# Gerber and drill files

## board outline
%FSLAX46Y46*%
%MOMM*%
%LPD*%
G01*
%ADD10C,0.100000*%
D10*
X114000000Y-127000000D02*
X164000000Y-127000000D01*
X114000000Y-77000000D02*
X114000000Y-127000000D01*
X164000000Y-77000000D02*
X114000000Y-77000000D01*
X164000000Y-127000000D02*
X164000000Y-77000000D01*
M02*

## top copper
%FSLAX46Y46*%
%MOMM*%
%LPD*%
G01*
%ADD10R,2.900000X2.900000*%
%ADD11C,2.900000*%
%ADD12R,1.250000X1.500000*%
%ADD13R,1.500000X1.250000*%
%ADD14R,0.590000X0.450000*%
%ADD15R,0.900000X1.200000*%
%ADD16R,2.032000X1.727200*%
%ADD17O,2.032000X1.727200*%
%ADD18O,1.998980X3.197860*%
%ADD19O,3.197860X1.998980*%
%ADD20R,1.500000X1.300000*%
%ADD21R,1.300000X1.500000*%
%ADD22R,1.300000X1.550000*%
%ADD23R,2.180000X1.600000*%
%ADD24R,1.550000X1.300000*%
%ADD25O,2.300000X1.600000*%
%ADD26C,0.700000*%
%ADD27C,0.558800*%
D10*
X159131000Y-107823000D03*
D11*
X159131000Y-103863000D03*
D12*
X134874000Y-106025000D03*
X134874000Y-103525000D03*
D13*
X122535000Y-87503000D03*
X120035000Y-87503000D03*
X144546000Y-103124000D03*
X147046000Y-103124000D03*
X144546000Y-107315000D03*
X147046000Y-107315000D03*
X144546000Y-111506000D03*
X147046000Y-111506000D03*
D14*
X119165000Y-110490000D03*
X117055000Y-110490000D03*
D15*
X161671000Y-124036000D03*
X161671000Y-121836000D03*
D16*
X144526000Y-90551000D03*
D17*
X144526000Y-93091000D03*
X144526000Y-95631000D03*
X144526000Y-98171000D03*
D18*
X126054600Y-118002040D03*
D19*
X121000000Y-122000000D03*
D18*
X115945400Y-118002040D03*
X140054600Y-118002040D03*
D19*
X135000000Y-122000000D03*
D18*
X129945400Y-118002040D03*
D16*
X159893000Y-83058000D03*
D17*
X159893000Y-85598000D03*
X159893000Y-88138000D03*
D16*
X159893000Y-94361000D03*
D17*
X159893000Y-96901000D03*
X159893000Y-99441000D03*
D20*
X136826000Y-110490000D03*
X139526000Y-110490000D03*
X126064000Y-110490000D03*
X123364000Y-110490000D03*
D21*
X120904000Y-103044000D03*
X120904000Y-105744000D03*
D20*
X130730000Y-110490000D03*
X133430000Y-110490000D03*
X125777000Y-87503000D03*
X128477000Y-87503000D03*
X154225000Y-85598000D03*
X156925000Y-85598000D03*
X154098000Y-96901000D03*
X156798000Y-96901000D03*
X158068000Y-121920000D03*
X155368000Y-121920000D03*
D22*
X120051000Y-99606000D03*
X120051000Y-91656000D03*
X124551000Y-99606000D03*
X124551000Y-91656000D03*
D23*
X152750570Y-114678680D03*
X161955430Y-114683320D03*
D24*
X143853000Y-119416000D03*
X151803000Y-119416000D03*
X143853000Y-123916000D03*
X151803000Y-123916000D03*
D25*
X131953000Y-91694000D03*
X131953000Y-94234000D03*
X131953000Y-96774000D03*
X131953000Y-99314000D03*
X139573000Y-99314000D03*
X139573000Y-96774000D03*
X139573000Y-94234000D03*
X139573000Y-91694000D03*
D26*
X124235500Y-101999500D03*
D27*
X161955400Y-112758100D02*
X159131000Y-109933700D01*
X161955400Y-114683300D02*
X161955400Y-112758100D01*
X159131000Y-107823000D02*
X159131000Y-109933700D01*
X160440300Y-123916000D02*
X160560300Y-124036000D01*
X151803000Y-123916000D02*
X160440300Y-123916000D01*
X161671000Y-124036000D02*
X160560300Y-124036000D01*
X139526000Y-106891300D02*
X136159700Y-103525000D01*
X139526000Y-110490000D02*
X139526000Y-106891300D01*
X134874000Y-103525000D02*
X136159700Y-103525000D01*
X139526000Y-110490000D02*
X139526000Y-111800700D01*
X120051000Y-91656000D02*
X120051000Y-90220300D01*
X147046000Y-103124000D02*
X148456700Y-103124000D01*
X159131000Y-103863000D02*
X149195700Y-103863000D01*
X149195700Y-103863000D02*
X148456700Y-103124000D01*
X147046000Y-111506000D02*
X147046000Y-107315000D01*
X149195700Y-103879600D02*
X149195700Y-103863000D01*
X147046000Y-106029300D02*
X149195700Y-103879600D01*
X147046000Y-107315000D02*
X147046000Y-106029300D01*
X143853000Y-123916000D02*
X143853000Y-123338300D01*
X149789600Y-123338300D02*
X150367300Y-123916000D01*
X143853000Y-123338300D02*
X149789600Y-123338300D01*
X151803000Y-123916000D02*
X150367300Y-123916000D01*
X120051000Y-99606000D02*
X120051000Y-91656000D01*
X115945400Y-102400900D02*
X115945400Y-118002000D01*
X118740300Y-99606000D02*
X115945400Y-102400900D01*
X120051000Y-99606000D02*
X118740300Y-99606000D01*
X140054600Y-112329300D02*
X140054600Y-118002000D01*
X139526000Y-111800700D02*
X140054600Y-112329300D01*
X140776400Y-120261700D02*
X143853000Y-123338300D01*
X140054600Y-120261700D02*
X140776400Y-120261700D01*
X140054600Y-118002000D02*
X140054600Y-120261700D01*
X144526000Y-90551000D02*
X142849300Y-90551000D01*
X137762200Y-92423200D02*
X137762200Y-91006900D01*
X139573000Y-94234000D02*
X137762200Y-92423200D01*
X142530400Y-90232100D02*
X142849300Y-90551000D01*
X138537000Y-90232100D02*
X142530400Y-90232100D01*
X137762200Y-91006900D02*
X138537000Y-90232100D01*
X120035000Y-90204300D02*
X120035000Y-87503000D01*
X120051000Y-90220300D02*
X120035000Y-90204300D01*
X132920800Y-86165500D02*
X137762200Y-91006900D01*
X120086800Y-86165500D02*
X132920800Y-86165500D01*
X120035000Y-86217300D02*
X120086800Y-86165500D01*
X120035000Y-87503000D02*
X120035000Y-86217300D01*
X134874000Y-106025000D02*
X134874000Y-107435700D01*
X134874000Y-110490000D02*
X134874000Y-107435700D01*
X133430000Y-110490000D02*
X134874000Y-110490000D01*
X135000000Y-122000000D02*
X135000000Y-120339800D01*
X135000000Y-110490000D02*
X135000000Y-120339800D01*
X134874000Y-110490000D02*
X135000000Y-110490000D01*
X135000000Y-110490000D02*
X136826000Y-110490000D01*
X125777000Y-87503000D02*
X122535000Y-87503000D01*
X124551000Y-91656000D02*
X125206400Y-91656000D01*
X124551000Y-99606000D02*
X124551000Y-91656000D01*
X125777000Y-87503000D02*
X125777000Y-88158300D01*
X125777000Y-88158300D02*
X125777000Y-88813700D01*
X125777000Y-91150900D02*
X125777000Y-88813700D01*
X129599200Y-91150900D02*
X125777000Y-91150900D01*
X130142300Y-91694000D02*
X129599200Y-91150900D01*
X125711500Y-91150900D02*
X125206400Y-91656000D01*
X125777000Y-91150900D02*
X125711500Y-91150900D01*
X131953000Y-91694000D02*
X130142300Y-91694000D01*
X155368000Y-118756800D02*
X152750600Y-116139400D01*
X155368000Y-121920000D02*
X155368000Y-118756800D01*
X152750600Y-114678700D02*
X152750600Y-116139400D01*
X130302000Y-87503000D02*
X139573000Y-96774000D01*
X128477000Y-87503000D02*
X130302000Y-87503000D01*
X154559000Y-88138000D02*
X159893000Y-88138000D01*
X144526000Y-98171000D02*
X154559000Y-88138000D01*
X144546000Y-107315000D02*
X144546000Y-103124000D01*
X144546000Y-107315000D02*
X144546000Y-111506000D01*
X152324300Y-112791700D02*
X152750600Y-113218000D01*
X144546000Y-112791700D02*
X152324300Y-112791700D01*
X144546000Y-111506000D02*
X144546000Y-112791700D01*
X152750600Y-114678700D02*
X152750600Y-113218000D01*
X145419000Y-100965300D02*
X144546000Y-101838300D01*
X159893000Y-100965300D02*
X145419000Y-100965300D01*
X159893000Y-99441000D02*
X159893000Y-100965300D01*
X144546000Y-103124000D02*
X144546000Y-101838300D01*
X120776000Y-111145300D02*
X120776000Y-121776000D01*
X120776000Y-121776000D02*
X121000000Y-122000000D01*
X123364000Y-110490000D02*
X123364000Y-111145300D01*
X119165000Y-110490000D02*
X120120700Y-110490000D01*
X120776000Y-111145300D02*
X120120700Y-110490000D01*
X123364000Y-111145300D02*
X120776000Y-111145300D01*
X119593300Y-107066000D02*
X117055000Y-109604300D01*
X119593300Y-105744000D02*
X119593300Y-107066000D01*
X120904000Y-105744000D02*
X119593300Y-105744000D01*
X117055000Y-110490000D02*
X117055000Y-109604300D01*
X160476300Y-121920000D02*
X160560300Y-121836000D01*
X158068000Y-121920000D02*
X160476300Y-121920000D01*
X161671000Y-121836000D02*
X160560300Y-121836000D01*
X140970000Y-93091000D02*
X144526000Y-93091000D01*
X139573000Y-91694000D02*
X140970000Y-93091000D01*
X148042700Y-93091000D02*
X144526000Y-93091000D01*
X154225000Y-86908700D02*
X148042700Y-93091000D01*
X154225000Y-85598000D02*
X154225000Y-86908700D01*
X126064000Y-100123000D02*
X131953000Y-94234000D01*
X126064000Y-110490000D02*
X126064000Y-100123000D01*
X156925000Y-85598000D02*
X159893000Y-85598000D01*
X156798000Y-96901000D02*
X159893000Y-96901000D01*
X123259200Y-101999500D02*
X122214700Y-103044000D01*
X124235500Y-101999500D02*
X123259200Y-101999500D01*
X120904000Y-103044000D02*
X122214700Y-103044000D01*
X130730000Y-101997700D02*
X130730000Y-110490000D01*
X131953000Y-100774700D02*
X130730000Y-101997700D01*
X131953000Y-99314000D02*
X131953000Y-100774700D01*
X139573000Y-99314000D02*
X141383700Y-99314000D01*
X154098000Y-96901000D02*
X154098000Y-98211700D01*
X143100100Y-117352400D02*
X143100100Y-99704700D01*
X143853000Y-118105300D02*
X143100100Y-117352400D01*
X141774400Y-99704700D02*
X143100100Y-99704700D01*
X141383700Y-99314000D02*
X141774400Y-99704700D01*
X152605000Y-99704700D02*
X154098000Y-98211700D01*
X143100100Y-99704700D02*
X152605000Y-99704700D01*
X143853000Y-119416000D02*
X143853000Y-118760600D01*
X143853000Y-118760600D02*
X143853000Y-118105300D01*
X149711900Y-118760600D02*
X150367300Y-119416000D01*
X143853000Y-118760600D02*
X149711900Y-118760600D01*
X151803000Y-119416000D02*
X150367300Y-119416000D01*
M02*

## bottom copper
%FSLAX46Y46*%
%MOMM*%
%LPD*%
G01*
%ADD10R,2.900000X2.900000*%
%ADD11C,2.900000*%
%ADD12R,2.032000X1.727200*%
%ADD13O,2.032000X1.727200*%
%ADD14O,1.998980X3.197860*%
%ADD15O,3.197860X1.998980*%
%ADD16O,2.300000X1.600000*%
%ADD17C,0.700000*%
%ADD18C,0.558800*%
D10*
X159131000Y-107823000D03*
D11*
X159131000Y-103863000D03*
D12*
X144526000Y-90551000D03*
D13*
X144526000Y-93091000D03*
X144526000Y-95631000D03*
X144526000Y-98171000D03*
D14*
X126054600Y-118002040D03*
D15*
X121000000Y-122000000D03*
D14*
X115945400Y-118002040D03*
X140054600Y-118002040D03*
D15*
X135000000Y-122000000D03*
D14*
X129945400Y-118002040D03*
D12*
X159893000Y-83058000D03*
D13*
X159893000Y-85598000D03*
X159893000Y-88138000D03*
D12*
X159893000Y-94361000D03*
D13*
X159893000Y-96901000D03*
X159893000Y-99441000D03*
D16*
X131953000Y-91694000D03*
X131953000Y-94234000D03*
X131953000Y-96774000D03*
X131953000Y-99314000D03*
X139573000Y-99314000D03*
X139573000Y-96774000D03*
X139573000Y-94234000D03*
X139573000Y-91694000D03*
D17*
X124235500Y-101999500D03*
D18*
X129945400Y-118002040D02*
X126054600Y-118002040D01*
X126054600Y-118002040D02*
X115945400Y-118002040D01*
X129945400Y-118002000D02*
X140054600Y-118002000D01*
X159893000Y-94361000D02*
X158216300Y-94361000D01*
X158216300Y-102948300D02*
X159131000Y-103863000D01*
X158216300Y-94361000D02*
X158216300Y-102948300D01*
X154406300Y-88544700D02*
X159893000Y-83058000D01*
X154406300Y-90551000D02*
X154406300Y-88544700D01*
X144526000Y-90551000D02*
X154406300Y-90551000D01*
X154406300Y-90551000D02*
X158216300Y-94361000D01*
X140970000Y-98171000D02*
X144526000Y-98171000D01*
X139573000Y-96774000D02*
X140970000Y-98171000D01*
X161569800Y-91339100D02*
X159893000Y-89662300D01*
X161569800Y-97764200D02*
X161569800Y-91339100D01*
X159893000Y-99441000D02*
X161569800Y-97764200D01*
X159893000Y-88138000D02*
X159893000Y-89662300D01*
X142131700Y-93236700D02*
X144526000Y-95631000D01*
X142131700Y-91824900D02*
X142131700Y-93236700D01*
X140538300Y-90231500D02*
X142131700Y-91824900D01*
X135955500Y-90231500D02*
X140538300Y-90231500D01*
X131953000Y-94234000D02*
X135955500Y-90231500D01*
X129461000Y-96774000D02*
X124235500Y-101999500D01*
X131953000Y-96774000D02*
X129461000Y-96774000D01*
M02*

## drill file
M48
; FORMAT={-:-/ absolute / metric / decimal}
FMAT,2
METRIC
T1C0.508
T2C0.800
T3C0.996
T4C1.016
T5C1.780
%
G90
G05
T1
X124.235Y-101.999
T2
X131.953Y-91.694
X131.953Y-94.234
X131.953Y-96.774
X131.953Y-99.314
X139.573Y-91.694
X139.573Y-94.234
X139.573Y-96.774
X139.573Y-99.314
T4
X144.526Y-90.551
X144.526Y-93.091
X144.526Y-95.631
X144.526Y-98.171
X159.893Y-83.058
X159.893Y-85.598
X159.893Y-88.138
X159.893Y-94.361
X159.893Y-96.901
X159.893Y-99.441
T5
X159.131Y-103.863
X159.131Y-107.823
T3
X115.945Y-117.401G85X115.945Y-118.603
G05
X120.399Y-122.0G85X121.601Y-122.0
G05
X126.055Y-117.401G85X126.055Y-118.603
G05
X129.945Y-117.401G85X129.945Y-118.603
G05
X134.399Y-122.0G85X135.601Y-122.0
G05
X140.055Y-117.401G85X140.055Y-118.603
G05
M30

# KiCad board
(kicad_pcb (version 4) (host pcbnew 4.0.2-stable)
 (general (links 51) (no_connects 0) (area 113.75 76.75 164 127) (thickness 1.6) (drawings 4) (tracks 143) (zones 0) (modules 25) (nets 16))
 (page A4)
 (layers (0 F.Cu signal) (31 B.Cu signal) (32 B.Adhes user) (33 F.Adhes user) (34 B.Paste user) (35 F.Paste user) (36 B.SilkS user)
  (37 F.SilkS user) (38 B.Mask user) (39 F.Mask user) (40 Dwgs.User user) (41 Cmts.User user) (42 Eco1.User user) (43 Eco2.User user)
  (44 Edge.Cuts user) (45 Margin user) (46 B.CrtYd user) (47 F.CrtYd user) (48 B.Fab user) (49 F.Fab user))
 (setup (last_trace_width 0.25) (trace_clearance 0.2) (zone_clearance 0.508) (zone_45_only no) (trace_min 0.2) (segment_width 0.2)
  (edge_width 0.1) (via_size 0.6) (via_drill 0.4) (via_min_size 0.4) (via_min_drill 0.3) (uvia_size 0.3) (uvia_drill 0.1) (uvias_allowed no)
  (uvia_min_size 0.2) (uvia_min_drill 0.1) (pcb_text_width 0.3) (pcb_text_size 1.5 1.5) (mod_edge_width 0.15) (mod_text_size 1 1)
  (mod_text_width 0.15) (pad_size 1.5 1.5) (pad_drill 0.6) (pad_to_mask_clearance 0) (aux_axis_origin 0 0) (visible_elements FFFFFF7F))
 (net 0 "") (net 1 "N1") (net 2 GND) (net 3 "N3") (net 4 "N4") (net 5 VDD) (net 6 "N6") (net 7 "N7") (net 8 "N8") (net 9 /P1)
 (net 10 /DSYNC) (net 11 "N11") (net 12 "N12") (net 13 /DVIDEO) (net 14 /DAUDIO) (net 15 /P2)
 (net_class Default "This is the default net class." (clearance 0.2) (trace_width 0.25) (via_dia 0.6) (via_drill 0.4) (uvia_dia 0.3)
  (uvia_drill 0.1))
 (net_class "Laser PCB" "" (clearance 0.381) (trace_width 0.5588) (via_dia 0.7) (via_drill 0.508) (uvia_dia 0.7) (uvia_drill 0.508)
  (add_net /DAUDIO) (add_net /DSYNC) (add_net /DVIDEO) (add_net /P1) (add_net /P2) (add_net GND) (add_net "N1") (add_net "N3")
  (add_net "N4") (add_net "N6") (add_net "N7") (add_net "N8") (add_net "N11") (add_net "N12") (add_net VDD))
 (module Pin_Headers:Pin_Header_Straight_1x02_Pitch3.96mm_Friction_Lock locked (layer F.Cu) (at 159.131 107.823 90)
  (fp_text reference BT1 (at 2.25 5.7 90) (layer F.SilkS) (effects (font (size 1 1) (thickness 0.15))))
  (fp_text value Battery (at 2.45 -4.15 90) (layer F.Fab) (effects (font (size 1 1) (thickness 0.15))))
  (pad 1 thru_hole rect (at 0 0 90) (size 2.9 2.9) (drill 1.78) (layers *.Cu *.Mask F.SilkS) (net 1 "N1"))
  (pad 2 thru_hole circle (at 3.96 0 90) (size 2.9 2.9) (drill 1.78) (layers *.Cu *.Mask F.SilkS) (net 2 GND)))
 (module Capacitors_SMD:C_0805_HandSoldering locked (layer F.Cu) (at 134.874 104.775 90)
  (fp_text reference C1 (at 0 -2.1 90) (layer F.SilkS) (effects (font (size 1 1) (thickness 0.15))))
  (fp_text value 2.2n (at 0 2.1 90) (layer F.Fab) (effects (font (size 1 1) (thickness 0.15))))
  (pad 1 smd rect (at -1.25 0 90) (size 1.5 1.25) (layers F.Cu F.Paste F.Mask) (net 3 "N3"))
  (pad 2 smd rect (at 1.25 0 90) (size 1.5 1.25) (layers F.Cu F.Paste F.Mask) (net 2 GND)))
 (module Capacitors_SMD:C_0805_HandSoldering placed (layer F.Cu) (at 121.285 87.503 180)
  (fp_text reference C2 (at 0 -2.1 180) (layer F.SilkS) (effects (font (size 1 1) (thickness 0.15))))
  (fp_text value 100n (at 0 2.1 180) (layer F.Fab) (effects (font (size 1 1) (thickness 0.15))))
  (pad 1 smd rect (at -1.25 0 180) (size 1.5 1.25) (layers F.Cu F.Paste F.Mask) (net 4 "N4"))
  (pad 2 smd rect (at 1.25 0 180) (size 1.5 1.25) (layers F.Cu F.Paste F.Mask) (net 2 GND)))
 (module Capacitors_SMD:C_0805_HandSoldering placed (layer F.Cu) (at 145.796 103.124)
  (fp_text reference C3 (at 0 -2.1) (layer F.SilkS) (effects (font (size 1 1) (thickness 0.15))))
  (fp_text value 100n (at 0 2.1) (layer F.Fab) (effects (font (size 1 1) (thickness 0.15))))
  (pad 1 smd rect (at -1.25 0) (size 1.5 1.25) (layers F.Cu F.Paste F.Mask) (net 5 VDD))
  (pad 2 smd rect (at 1.25 0) (size 1.5 1.25) (layers F.Cu F.Paste F.Mask) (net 2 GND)))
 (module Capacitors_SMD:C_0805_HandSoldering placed (layer F.Cu) (at 145.796 107.315)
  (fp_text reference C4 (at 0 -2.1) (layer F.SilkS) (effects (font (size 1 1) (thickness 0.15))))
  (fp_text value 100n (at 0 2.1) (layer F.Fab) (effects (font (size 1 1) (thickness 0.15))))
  (pad 1 smd rect (at -1.25 0) (size 1.5 1.25) (layers F.Cu F.Paste F.Mask) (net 5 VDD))
  (pad 2 smd rect (at 1.25 0) (size 1.5 1.25) (layers F.Cu F.Paste F.Mask) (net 2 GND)))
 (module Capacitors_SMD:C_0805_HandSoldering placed (layer F.Cu) (at 145.796 111.506)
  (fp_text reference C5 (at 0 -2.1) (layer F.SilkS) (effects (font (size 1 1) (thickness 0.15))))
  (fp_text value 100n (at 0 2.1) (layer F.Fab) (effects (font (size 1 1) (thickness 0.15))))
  (pad 1 smd rect (at -1.25 0) (size 1.5 1.25) (layers F.Cu F.Paste F.Mask) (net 5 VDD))
  (pad 2 smd rect (at 1.25 0) (size 1.5 1.25) (layers F.Cu F.Paste F.Mask) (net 2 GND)))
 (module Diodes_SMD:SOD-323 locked (layer F.Cu) (at 118.11 110.49 180)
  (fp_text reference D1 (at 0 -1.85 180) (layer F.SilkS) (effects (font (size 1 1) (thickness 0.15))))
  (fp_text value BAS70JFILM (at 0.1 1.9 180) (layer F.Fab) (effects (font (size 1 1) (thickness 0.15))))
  (pad 1 smd rect (at -1.055 0 180) (size 0.59 0.45) (layers F.Cu F.Paste F.Mask) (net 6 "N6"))
  (pad 2 smd rect (at 1.055 0 180) (size 0.59 0.45) (layers F.Cu F.Paste F.Mask) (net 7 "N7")))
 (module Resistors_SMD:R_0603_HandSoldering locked (layer F.Cu) (at 161.671 122.936 90)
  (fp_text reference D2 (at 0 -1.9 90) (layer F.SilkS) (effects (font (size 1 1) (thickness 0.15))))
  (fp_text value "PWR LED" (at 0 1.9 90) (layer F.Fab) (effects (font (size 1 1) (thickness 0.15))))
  (pad 1 smd rect (at -1.1 0 90) (size 1.2 0.9) (layers F.Cu F.Paste F.Mask) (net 2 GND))
  (pad 2 smd rect (at 1.1 0 90) (size 1.2 0.9) (layers F.Cu F.Paste F.Mask) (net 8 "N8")))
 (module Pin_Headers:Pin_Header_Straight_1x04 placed (layer F.Cu) (at 144.526 90.551)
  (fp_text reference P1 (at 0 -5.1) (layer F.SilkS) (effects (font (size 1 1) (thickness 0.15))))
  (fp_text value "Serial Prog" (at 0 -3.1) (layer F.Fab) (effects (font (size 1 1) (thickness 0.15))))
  (pad 1 thru_hole rect (at 0 0) (size 2.032 1.7272) (drill 1.016) (layers *.Cu *.Mask F.SilkS) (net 2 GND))
  (pad 2 thru_hole oval (at 0 2.54) (size 2.032 1.7272) (drill 1.016) (layers *.Cu *.Mask F.SilkS) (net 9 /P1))
  (pad 3 thru_hole oval (at 0 5.08) (size 2.032 1.7272) (drill 1.016) (layers *.Cu *.Mask F.SilkS) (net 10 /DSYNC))
  (pad 4 thru_hole oval (at 0 7.62) (size 2.032 1.7272) (drill 1.016) (layers *.Cu *.Mask F.SilkS) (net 5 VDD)))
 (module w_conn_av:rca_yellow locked (layer F.Cu) (at 121 122)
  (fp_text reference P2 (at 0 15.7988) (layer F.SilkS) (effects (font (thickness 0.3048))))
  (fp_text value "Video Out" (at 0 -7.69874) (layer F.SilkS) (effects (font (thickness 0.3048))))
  (pad 2 thru_hole oval (at 5.0546 -3.99796) (size 1.99898 3.19786) (drill oval 0.99568 2.1971) (layers *.Cu *.Mask F.SilkS) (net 2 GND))
  (pad 1 thru_hole oval (at 0 0) (size 3.19786 1.99898) (drill oval 2.1971 0.99568) (layers *.Cu *.Mask F.SilkS) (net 6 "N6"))
  (pad 2 thru_hole oval (at -5.0546 -3.99796) (size 1.99898 3.19786) (drill oval 0.99568 2.1971) (layers *.Cu *.Mask F.SilkS) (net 2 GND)))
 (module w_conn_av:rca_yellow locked (layer F.Cu) (at 135 122)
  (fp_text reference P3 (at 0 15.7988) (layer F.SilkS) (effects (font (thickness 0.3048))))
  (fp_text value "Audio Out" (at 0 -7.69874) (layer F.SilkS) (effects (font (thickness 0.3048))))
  (pad 2 thru_hole oval (at 5.0546 -3.99796) (size 1.99898 3.19786) (drill oval 0.99568 2.1971) (layers *.Cu *.Mask F.SilkS) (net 2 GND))
  (pad 1 thru_hole oval (at 0 0) (size 3.19786 1.99898) (drill oval 2.1971 0.99568) (layers *.Cu *.Mask F.SilkS) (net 3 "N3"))
  (pad 2 thru_hole oval (at -5.0546 -3.99796) (size 1.99898 3.19786) (drill oval 0.99568 2.1971) (layers *.Cu *.Mask F.SilkS) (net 2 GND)))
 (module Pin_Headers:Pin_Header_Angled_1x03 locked (layer F.Cu) (at 159.893 83.058)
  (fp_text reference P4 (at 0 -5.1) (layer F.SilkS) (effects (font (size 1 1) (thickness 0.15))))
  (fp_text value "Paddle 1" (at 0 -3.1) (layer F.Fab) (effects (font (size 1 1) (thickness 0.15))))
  (pad 1 thru_hole rect (at 0 0) (size 2.032 1.7272) (drill 1.016) (layers *.Cu *.Mask F.SilkS) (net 2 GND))
  (pad 2 thru_hole oval (at 0 2.54) (size 2.032 1.7272) (drill 1.016) (layers *.Cu *.Mask F.SilkS) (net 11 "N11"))
  (pad 3 thru_hole oval (at 0 5.08) (size 2.032 1.7272) (drill 1.016) (layers *.Cu *.Mask F.SilkS) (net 5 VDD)))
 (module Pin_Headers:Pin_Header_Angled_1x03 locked (layer F.Cu) (at 159.893 94.361)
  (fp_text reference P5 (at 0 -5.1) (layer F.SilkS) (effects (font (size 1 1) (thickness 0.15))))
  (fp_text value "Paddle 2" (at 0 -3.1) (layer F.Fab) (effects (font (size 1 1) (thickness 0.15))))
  (pad 1 thru_hole rect (at 0 0) (size 2.032 1.7272) (drill 1.016) (layers *.Cu *.Mask F.SilkS) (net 2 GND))
  (pad 2 thru_hole oval (at 0 2.54) (size 2.032 1.7272) (drill 1.016) (layers *.Cu *.Mask F.SilkS) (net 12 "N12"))
  (pad 3 thru_hole oval (at 0 5.08) (size 2.032 1.7272) (drill 1.016) (layers *.Cu *.Mask F.SilkS) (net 5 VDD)))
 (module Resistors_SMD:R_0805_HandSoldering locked (layer F.Cu) (at 138.176 110.49)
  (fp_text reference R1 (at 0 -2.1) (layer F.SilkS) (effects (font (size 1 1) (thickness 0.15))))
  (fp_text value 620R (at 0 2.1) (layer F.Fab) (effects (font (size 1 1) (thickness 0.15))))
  (pad 1 smd rect (at -1.35 0) (size 1.5 1.3) (layers F.Cu F.Paste F.Mask) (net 3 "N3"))
  (pad 2 smd rect (at 1.35 0) (size 1.5 1.3) (layers F.Cu F.Paste F.Mask) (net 2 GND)))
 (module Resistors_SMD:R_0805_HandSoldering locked (layer F.Cu) (at 124.714 110.49 180)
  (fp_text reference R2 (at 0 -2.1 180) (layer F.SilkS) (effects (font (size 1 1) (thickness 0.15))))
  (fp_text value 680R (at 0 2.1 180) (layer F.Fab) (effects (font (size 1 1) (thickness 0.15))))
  (pad 1 smd rect (at -1.35 0 180) (size 1.5 1.3) (layers F.Cu F.Paste F.Mask) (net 10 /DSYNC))
  (pad 2 smd rect (at 1.35 0 180) (size 1.5 1.3) (layers F.Cu F.Paste F.Mask) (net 6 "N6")))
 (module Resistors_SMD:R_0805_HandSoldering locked (layer F.Cu) (at 120.904 104.394 270)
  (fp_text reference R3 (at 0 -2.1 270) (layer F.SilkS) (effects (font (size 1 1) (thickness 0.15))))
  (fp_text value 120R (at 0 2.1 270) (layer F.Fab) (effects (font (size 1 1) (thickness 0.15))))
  (pad 1 smd rect (at -1.35 0 270) (size 1.5 1.3) (layers F.Cu F.Paste F.Mask) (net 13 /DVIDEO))
  (pad 2 smd rect (at 1.35 0 270) (size 1.5 1.3) (layers F.Cu F.Paste F.Mask) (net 7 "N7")))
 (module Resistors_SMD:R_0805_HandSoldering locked (layer F.Cu) (at 132.08 110.49)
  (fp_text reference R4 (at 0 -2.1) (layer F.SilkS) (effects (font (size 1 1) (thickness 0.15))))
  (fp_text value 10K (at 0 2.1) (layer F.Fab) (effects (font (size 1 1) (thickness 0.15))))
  (pad 1 smd rect (at -1.35 0) (size 1.5 1.3) (layers F.Cu F.Paste F.Mask) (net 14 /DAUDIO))
  (pad 2 smd rect (at 1.35 0) (size 1.5 1.3) (layers F.Cu F.Paste F.Mask) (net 3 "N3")))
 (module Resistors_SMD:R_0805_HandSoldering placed (layer F.Cu) (at 127.127 87.503)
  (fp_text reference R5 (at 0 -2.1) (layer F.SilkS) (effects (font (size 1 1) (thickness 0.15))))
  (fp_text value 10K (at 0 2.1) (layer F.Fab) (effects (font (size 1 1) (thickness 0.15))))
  (pad 1 smd rect (at -1.35 0) (size 1.5 1.3) (layers F.Cu F.Paste F.Mask) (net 4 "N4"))
  (pad 2 smd rect (at 1.35 0) (size 1.5 1.3) (layers F.Cu F.Paste F.Mask) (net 5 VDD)))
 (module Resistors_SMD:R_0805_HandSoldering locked (layer F.Cu) (at 155.575 85.598)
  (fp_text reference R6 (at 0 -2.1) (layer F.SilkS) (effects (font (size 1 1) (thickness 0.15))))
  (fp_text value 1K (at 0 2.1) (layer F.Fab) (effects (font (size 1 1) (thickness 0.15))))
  (pad 1 smd rect (at -1.35 0) (size 1.5 1.3) (layers F.Cu F.Paste F.Mask) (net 9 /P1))
  (pad 2 smd rect (at 1.35 0) (size 1.5 1.3) (layers F.Cu F.Paste F.Mask) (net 11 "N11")))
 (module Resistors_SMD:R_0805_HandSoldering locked (layer F.Cu) (at 155.448 96.901)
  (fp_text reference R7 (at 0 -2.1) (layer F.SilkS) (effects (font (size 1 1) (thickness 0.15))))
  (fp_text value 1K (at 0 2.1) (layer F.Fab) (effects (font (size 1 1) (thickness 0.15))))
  (pad 1 smd rect (at -1.35 0) (size 1.5 1.3) (layers F.Cu F.Paste F.Mask) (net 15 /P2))
  (pad 2 smd rect (at 1.35 0) (size 1.5 1.3) (layers F.Cu F.Paste F.Mask) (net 12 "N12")))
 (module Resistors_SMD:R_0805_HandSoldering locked (layer F.Cu) (at 156.718 121.92 180)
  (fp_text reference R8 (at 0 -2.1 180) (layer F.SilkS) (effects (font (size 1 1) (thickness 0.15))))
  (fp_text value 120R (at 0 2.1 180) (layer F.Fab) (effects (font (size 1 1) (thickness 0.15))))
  (pad 1 smd rect (at -1.35 0 180) (size 1.5 1.3) (layers F.Cu F.Paste F.Mask) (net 8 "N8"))
  (pad 2 smd rect (at 1.35 0 180) (size 1.5 1.3) (layers F.Cu F.Paste F.Mask) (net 5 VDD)))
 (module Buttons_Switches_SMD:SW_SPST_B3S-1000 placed (layer F.Cu) (at 122.301 95.631 90)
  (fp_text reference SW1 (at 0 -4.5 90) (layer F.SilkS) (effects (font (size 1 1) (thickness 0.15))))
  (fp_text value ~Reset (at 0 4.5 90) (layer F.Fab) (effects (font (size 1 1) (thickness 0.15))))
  (pad 1 smd rect (at -3.975 -2.25 90) (size 1.55 1.3) (layers F.Cu F.Paste F.Mask) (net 2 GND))
  (pad 1 smd rect (at 3.975 -2.25 90) (size 1.55 1.3) (layers F.Cu F.Paste F.Mask) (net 2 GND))
  (pad 2 smd rect (at -3.975 2.25 90) (size 1.55 1.3) (layers F.Cu F.Paste F.Mask) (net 4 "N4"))
  (pad 2 smd rect (at 3.975 2.25 90) (size 1.55 1.3) (layers F.Cu F.Paste F.Mask) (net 4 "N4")))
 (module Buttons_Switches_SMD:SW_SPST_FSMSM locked (layer F.Cu) (at 157.353 114.681)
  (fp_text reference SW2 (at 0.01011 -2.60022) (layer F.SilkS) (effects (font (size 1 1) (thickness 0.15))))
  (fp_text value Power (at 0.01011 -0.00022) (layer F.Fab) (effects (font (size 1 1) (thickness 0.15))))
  (pad 1 smd rect (at -4.60243 -0.00232) (size 2.18 1.6) (layers F.Cu F.Paste F.Mask) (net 5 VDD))
  (pad 2 smd rect (at 4.60243 0.00232) (size 2.18 1.6) (layers F.Cu F.Paste F.Mask) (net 1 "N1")))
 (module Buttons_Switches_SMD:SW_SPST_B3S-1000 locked (layer F.Cu) (at 147.828 121.666)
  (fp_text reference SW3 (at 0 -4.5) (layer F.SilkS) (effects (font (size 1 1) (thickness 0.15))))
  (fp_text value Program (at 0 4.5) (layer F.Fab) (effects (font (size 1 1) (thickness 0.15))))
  (pad 1 smd rect (at -3.975 -2.25) (size 1.55 1.3) (layers F.Cu F.Paste F.Mask) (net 15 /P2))
  (pad 1 smd rect (at 3.975 -2.25) (size 1.55 1.3) (layers F.Cu F.Paste F.Mask) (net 15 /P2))
  (pad 2 smd rect (at -3.975 2.25) (size 1.55 1.3) (layers F.Cu F.Paste F.Mask) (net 2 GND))
  (pad 2 smd rect (at 3.975 2.25) (size 1.55 1.3) (layers F.Cu F.Paste F.Mask) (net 2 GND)))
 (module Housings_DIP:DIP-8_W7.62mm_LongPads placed (layer F.Cu) (at 131.953 91.694)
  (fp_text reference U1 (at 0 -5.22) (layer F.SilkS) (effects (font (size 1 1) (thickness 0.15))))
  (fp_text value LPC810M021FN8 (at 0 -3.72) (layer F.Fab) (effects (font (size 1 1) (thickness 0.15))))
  (pad 1 thru_hole oval (at 0 0) (size 2.3 1.6) (drill 0.8) (layers *.Cu *.Mask F.SilkS) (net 4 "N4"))
  (pad 2 thru_hole oval (at 0 2.54) (size 2.3 1.6) (drill 0.8) (layers *.Cu *.Mask F.SilkS) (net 10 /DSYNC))
  (pad 3 thru_hole oval (at 0 5.08) (size 2.3 1.6) (drill 0.8) (layers *.Cu *.Mask F.SilkS) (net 13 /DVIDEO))
  (pad 4 thru_hole oval (at 0 7.62) (size 2.3 1.6) (drill 0.8) (layers *.Cu *.Mask F.SilkS) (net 14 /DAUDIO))
  (pad 5 thru_hole oval (at 7.62 7.62) (size 2.3 1.6) (drill 0.8) (layers *.Cu *.Mask F.SilkS) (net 15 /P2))
  (pad 6 thru_hole oval (at 7.62 5.08) (size 2.3 1.6) (drill 0.8) (layers *.Cu *.Mask F.SilkS) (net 5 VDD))
  (pad 7 thru_hole oval (at 7.62 2.54) (size 2.3 1.6) (drill 0.8) (layers *.Cu *.Mask F.SilkS) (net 2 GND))
  (pad 8 thru_hole oval (at 7.62 0) (size 2.3 1.6) (drill 0.8) (layers *.Cu *.Mask F.SilkS) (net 9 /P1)))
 (gr_line (start 114 127) (end 164 127) (angle 90) (layer Edge.Cuts) (width 0.1))
 (gr_line (start 114 77) (end 114 127) (angle 90) (layer Edge.Cuts) (width 0.1))
 (gr_line (start 164 77) (end 114 77) (angle 90) (layer Edge.Cuts) (width 0.1))
 (gr_line (start 164 127) (end 164 77) (angle 90) (layer Edge.Cuts) (width 0.1))
 (segment (start 161.9554 112.7581) (end 159.131 109.9337) (width 0.5588) (layer F.Cu) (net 1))
 (segment (start 161.9554 114.6833) (end 161.9554 112.7581) (width 0.5588) (layer F.Cu) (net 1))
 (segment (start 159.131 107.823) (end 159.131 109.9337) (width 0.5588) (layer F.Cu) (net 1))
 (segment (start 129.9454 118.00204) (end 126.0546 118.00204) (width 0.5588) (layer B.Cu) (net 2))
 (segment (start 126.0546 118.00204) (end 115.9454 118.00204) (width 0.5588) (layer B.Cu) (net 2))
 (segment (start 160.4403 123.916) (end 160.5603 124.036) (width 0.5588) (layer F.Cu) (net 2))
 (segment (start 151.803 123.916) (end 160.4403 123.916) (width 0.5588) (layer F.Cu) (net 2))
 (segment (start 161.671 124.036) (end 160.5603 124.036) (width 0.5588) (layer F.Cu) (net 2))
 (segment (start 139.526 106.8913) (end 136.1597 103.525) (width 0.5588) (layer F.Cu) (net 2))
 (segment (start 139.526 110.49) (end 139.526 106.8913) (width 0.5588) (layer F.Cu) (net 2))
 (segment (start 134.874 103.525) (end 136.1597 103.525) (width 0.5588) (layer F.Cu) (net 2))
 (segment (start 139.526 110.49) (end 139.526 111.8007) (width 0.5588) (layer F.Cu) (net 2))
 (segment (start 120.051 91.656) (end 120.051 90.2203) (width 0.5588) (layer F.Cu) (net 2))
 (segment (start 147.046 103.124) (end 148.4567 103.124) (width 0.5588) (layer F.Cu) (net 2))
 (segment (start 159.131 103.863) (end 149.1957 103.863) (width 0.5588) (layer F.Cu) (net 2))
 (segment (start 149.1957 103.863) (end 148.4567 103.124) (width 0.5588) (layer F.Cu) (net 2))
 (segment (start 147.046 111.506) (end 147.046 107.315) (width 0.5588) (layer F.Cu) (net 2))
 (segment (start 149.1957 103.8796) (end 149.1957 103.863) (width 0.5588) (layer F.Cu) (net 2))
 (segment (start 147.046 106.0293) (end 149.1957 103.8796) (width 0.5588) (layer F.Cu) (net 2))
 (segment (start 147.046 107.315) (end 147.046 106.0293) (width 0.5588) (layer F.Cu) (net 2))
 (segment (start 143.853 123.916) (end 143.853 123.3383) (width 0.5588) (layer F.Cu) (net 2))
 (segment (start 149.7896 123.3383) (end 150.3673 123.916) (width 0.5588) (layer F.Cu) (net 2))
 (segment (start 143.853 123.3383) (end 149.7896 123.3383) (width 0.5588) (layer F.Cu) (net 2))
 (segment (start 151.803 123.916) (end 150.3673 123.916) (width 0.5588) (layer F.Cu) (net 2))
 (segment (start 120.051 99.606) (end 120.051 91.656) (width 0.5588) (layer F.Cu) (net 2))
 (segment (start 115.9454 102.4009) (end 115.9454 118.002) (width 0.5588) (layer F.Cu) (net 2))
 (segment (start 118.7403 99.606) (end 115.9454 102.4009) (width 0.5588) (layer F.Cu) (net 2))
 (segment (start 120.051 99.606) (end 118.7403 99.606) (width 0.5588) (layer F.Cu) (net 2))
 (segment (start 140.0546 112.3293) (end 140.0546 118.002) (width 0.5588) (layer F.Cu) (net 2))
 (segment (start 139.526 111.8007) (end 140.0546 112.3293) (width 0.5588) (layer F.Cu) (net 2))
 (segment (start 140.7764 120.2617) (end 143.853 123.3383) (width 0.5588) (layer F.Cu) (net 2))
 (segment (start 140.0546 120.2617) (end 140.7764 120.2617) (width 0.5588) (layer F.Cu) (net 2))
 (segment (start 140.0546 118.002) (end 140.0546 120.2617) (width 0.5588) (layer F.Cu) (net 2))
 (segment (start 129.9454 118.002) (end 140.0546 118.002) (width 0.5588) (layer B.Cu) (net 2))
 (segment (start 159.893 94.361) (end 158.2163 94.361) (width 0.5588) (layer B.Cu) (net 2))
 (segment (start 158.2163 102.9483) (end 159.131 103.863) (width 0.5588) (layer B.Cu) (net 2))
 (segment (start 158.2163 94.361) (end 158.2163 102.9483) (width 0.5588) (layer B.Cu) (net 2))
 (segment (start 144.526 90.551) (end 142.8493 90.551) (width 0.5588) (layer F.Cu) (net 2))
 (segment (start 137.7622 92.4232) (end 137.7622 91.0069) (width 0.5588) (layer F.Cu) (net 2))
 (segment (start 139.573 94.234) (end 137.7622 92.4232) (width 0.5588) (layer F.Cu) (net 2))
 (segment (start 142.5304 90.2321) (end 142.8493 90.551) (width 0.5588) (layer F.Cu) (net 2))
 (segment (start 138.537 90.2321) (end 142.5304 90.2321) (width 0.5588) (layer F.Cu) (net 2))
 (segment (start 137.7622 91.0069) (end 138.537 90.2321) (width 0.5588) (layer F.Cu) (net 2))
 (segment (start 120.035 90.2043) (end 120.035 87.503) (width 0.5588) (layer F.Cu) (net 2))
 (segment (start 120.051 90.2203) (end 120.035 90.2043) (width 0.5588) (layer F.Cu) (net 2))
 (segment (start 132.9208 86.1655) (end 137.7622 91.0069) (width 0.5588) (layer F.Cu) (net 2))
 (segment (start 120.0868 86.1655) (end 132.9208 86.1655) (width 0.5588) (layer F.Cu) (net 2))
 (segment (start 120.035 86.2173) (end 120.0868 86.1655) (width 0.5588) (layer F.Cu) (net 2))
 (segment (start 120.035 87.503) (end 120.035 86.2173) (width 0.5588) (layer F.Cu) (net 2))
 (segment (start 154.4063 88.5447) (end 159.893 83.058) (width 0.5588) (layer B.Cu) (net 2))
 (segment (start 154.4063 90.551) (end 154.4063 88.5447) (width 0.5588) (layer B.Cu) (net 2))
 (segment (start 144.526 90.551) (end 154.4063 90.551) (width 0.5588) (layer B.Cu) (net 2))
 (segment (start 154.4063 90.551) (end 158.2163 94.361) (width 0.5588) (layer B.Cu) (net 2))
 (segment (start 134.874 106.025) (end 134.874 107.4357) (width 0.5588) (layer F.Cu) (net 3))
 (segment (start 134.874 110.49) (end 134.874 107.4357) (width 0.5588) (layer F.Cu) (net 3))
 (segment (start 133.43 110.49) (end 134.874 110.49) (width 0.5588) (layer F.Cu) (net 3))
 (segment (start 135 122) (end 135 120.3398) (width 0.5588) (layer F.Cu) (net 3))
 (segment (start 135 110.49) (end 135 120.3398) (width 0.5588) (layer F.Cu) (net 3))
 (segment (start 134.874 110.49) (end 135 110.49) (width 0.5588) (layer F.Cu) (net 3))
 (segment (start 135 110.49) (end 136.826 110.49) (width 0.5588) (layer F.Cu) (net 3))
 (segment (start 125.777 87.503) (end 122.535 87.503) (width 0.5588) (layer F.Cu) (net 4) (status C00000))
 (segment (start 124.551 91.656) (end 125.2064 91.656) (width 0.5588) (layer F.Cu) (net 4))
 (segment (start 124.551 99.606) (end 124.551 91.656) (width 0.5588) (layer F.Cu) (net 4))
 (segment (start 125.777 87.503) (end 125.777 88.1583) (width 0.5588) (layer F.Cu) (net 4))
 (segment (start 125.777 88.1583) (end 125.777 88.8137) (width 0.5588) (layer F.Cu) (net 4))
 (segment (start 125.777 91.1509) (end 125.777 88.8137) (width 0.5588) (layer F.Cu) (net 4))
 (segment (start 129.5992 91.1509) (end 125.777 91.1509) (width 0.5588) (layer F.Cu) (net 4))
 (segment (start 130.1423 91.694) (end 129.5992 91.1509) (width 0.5588) (layer F.Cu) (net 4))
 (segment (start 125.7115 91.1509) (end 125.2064 91.656) (width 0.5588) (layer F.Cu) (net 4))
 (segment (start 125.777 91.1509) (end 125.7115 91.1509) (width 0.5588) (layer F.Cu) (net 4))
 (segment (start 131.953 91.694) (end 130.1423 91.694) (width 0.5588) (layer F.Cu) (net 4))
 (segment (start 155.368 118.7568) (end 152.7506 116.1394) (width 0.5588) (layer F.Cu) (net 5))
 (segment (start 155.368 121.92) (end 155.368 118.7568) (width 0.5588) (layer F.Cu) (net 5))
 (segment (start 152.7506 114.6787) (end 152.7506 116.1394) (width 0.5588) (layer F.Cu) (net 5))
 (segment (start 130.302 87.503) (end 139.573 96.774) (width 0.5588) (layer F.Cu) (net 5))
 (segment (start 128.477 87.503) (end 130.302 87.503) (width 0.5588) (layer F.Cu) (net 5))
 (segment (start 140.97 98.171) (end 144.526 98.171) (width 0.5588) (layer B.Cu) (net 5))
 (segment (start 139.573 96.774) (end 140.97 98.171) (width 0.5588) (layer B.Cu) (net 5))
 (segment (start 161.5698 91.3391) (end 159.893 89.6623) (width 0.5588) (layer B.Cu) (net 5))
 (segment (start 161.5698 97.7642) (end 161.5698 91.3391) (width 0.5588) (layer B.Cu) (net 5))
 (segment (start 159.893 99.441) (end 161.5698 97.7642) (width 0.5588) (layer B.Cu) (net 5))
 (segment (start 159.893 88.138) (end 159.893 89.6623) (width 0.5588) (layer B.Cu) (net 5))
 (segment (start 154.559 88.138) (end 159.893 88.138) (width 0.5588) (layer F.Cu) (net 5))
 (segment (start 144.526 98.171) (end 154.559 88.138) (width 0.5588) (layer F.Cu) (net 5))
 (segment (start 144.546 107.315) (end 144.546 103.124) (width 0.5588) (layer F.Cu) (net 5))
 (segment (start 144.546 107.315) (end 144.546 111.506) (width 0.5588) (layer F.Cu) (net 5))
 (segment (start 152.3243 112.7917) (end 152.7506 113.218) (width 0.5588) (layer F.Cu) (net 5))
 (segment (start 144.546 112.7917) (end 152.3243 112.7917) (width 0.5588) (layer F.Cu) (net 5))
 (segment (start 144.546 111.506) (end 144.546 112.7917) (width 0.5588) (layer F.Cu) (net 5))
 (segment (start 152.7506 114.6787) (end 152.7506 113.218) (width 0.5588) (layer F.Cu) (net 5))
 (segment (start 145.419 100.9653) (end 144.546 101.8383) (width 0.5588) (layer F.Cu) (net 5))
 (segment (start 159.893 100.9653) (end 145.419 100.9653) (width 0.5588) (layer F.Cu) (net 5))
 (segment (start 159.893 99.441) (end 159.893 100.9653) (width 0.5588) (layer F.Cu) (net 5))
 (segment (start 144.546 103.124) (end 144.546 101.8383) (width 0.5588) (layer F.Cu) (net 5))
 (segment (start 120.776 111.1453) (end 120.776 121.776) (width 0.5588) (layer F.Cu) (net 6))
 (segment (start 120.776 121.776) (end 121 122) (width 0.5588) (layer F.Cu) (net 6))
 (segment (start 123.364 110.49) (end 123.364 111.1453) (width 0.5588) (layer F.Cu) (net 6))
 (segment (start 119.165 110.49) (end 120.1207 110.49) (width 0.5588) (layer F.Cu) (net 6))
 (segment (start 120.776 111.1453) (end 120.1207 110.49) (width 0.5588) (layer F.Cu) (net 6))
 (segment (start 123.364 111.1453) (end 120.776 111.1453) (width 0.5588) (layer F.Cu) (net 6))
 (segment (start 119.5933 107.066) (end 117.055 109.6043) (width 0.5588) (layer F.Cu) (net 7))
 (segment (start 119.5933 105.744) (end 119.5933 107.066) (width 0.5588) (layer F.Cu) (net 7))
 (segment (start 120.904 105.744) (end 119.5933 105.744) (width 0.5588) (layer F.Cu) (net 7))
 (segment (start 117.055 110.49) (end 117.055 109.6043) (width 0.5588) (layer F.Cu) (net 7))
 (segment (start 160.4763 121.92) (end 160.5603 121.836) (width 0.5588) (layer F.Cu) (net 8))
 (segment (start 158.068 121.92) (end 160.4763 121.92) (width 0.5588) (layer F.Cu) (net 8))
 (segment (start 161.671 121.836) (end 160.5603 121.836) (width 0.5588) (layer F.Cu) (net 8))
 (segment (start 140.97 93.091) (end 144.526 93.091) (width 0.5588) (layer F.Cu) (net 9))
 (segment (start 139.573 91.694) (end 140.97 93.091) (width 0.5588) (layer F.Cu) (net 9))
 (segment (start 148.0427 93.091) (end 144.526 93.091) (width 0.5588) (layer F.Cu) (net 9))
 (segment (start 154.225 86.9087) (end 148.0427 93.091) (width 0.5588) (layer F.Cu) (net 9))
 (segment (start 154.225 85.598) (end 154.225 86.9087) (width 0.5588) (layer F.Cu) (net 9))
 (segment (start 142.1317 93.2367) (end 144.526 95.631) (width 0.5588) (layer B.Cu) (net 10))
 (segment (start 142.1317 91.8249) (end 142.1317 93.2367) (width 0.5588) (layer B.Cu) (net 10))
 (segment (start 140.5383 90.2315) (end 142.1317 91.8249) (width 0.5588) (layer B.Cu) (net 10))
 (segment (start 135.9555 90.2315) (end 140.5383 90.2315) (width 0.5588) (layer B.Cu) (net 10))
 (segment (start 131.953 94.234) (end 135.9555 90.2315) (width 0.5588) (layer B.Cu) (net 10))
 (segment (start 126.064 100.123) (end 131.953 94.234) (width 0.5588) (layer F.Cu) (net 10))
 (segment (start 126.064 110.49) (end 126.064 100.123) (width 0.5588) (layer F.Cu) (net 10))
 (segment (start 156.925 85.598) (end 159.893 85.598) (width 0.5588) (layer F.Cu) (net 11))
 (segment (start 156.798 96.901) (end 159.893 96.901) (width 0.5588) (layer F.Cu) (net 12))
 (via (at 124.2355 101.9995) (size 0.7) (drill 0.508) (layers F.Cu B.Cu) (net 13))
 (segment (start 129.461 96.774) (end 124.2355 101.9995) (width 0.5588) (layer B.Cu) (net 13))
 (segment (start 131.953 96.774) (end 129.461 96.774) (width 0.5588) (layer B.Cu) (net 13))
 (segment (start 123.2592 101.9995) (end 122.2147 103.044) (width 0.5588) (layer F.Cu) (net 13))
 (segment (start 124.2355 101.9995) (end 123.2592 101.9995) (width 0.5588) (layer F.Cu) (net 13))
 (segment (start 120.904 103.044) (end 122.2147 103.044) (width 0.5588) (layer F.Cu) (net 13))
 (segment (start 130.73 101.9977) (end 130.73 110.49) (width 0.5588) (layer F.Cu) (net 14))
 (segment (start 131.953 100.7747) (end 130.73 101.9977) (width 0.5588) (layer F.Cu) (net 14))
 (segment (start 131.953 99.314) (end 131.953 100.7747) (width 0.5588) (layer F.Cu) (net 14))
 (segment (start 139.573 99.314) (end 141.3837 99.314) (width 0.5588) (layer F.Cu) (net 15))
 (segment (start 154.098 96.901) (end 154.098 98.2117) (width 0.5588) (layer F.Cu) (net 15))
 (segment (start 143.1001 117.3524) (end 143.1001 99.7047) (width 0.5588) (layer F.Cu) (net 15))
 (segment (start 143.853 118.1053) (end 143.1001 117.3524) (width 0.5588) (layer F.Cu) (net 15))
 (segment (start 141.7744 99.7047) (end 143.1001 99.7047) (width 0.5588) (layer F.Cu) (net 15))
 (segment (start 141.3837 99.314) (end 141.7744 99.7047) (width 0.5588) (layer F.Cu) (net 15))
 (segment (start 152.605 99.7047) (end 154.098 98.2117) (width 0.5588) (layer F.Cu) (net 15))
 (segment (start 143.1001 99.7047) (end 152.605 99.7047) (width 0.5588) (layer F.Cu) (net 15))
 (segment (start 143.853 119.416) (end 143.853 118.7606) (width 0.5588) (layer F.Cu) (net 15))
 (segment (start 143.853 118.7606) (end 143.853 118.1053) (width 0.5588) (layer F.Cu) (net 15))
 (segment (start 149.7119 118.7606) (end 150.3673 119.416) (width 0.5588) (layer F.Cu) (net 15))
 (segment (start 143.853 118.7606) (end 149.7119 118.7606) (width 0.5588) (layer F.Cu) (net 15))
 (segment (start 151.803 119.416) (end 150.3673 119.416) (width 0.5588) (layer F.Cu) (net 15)))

